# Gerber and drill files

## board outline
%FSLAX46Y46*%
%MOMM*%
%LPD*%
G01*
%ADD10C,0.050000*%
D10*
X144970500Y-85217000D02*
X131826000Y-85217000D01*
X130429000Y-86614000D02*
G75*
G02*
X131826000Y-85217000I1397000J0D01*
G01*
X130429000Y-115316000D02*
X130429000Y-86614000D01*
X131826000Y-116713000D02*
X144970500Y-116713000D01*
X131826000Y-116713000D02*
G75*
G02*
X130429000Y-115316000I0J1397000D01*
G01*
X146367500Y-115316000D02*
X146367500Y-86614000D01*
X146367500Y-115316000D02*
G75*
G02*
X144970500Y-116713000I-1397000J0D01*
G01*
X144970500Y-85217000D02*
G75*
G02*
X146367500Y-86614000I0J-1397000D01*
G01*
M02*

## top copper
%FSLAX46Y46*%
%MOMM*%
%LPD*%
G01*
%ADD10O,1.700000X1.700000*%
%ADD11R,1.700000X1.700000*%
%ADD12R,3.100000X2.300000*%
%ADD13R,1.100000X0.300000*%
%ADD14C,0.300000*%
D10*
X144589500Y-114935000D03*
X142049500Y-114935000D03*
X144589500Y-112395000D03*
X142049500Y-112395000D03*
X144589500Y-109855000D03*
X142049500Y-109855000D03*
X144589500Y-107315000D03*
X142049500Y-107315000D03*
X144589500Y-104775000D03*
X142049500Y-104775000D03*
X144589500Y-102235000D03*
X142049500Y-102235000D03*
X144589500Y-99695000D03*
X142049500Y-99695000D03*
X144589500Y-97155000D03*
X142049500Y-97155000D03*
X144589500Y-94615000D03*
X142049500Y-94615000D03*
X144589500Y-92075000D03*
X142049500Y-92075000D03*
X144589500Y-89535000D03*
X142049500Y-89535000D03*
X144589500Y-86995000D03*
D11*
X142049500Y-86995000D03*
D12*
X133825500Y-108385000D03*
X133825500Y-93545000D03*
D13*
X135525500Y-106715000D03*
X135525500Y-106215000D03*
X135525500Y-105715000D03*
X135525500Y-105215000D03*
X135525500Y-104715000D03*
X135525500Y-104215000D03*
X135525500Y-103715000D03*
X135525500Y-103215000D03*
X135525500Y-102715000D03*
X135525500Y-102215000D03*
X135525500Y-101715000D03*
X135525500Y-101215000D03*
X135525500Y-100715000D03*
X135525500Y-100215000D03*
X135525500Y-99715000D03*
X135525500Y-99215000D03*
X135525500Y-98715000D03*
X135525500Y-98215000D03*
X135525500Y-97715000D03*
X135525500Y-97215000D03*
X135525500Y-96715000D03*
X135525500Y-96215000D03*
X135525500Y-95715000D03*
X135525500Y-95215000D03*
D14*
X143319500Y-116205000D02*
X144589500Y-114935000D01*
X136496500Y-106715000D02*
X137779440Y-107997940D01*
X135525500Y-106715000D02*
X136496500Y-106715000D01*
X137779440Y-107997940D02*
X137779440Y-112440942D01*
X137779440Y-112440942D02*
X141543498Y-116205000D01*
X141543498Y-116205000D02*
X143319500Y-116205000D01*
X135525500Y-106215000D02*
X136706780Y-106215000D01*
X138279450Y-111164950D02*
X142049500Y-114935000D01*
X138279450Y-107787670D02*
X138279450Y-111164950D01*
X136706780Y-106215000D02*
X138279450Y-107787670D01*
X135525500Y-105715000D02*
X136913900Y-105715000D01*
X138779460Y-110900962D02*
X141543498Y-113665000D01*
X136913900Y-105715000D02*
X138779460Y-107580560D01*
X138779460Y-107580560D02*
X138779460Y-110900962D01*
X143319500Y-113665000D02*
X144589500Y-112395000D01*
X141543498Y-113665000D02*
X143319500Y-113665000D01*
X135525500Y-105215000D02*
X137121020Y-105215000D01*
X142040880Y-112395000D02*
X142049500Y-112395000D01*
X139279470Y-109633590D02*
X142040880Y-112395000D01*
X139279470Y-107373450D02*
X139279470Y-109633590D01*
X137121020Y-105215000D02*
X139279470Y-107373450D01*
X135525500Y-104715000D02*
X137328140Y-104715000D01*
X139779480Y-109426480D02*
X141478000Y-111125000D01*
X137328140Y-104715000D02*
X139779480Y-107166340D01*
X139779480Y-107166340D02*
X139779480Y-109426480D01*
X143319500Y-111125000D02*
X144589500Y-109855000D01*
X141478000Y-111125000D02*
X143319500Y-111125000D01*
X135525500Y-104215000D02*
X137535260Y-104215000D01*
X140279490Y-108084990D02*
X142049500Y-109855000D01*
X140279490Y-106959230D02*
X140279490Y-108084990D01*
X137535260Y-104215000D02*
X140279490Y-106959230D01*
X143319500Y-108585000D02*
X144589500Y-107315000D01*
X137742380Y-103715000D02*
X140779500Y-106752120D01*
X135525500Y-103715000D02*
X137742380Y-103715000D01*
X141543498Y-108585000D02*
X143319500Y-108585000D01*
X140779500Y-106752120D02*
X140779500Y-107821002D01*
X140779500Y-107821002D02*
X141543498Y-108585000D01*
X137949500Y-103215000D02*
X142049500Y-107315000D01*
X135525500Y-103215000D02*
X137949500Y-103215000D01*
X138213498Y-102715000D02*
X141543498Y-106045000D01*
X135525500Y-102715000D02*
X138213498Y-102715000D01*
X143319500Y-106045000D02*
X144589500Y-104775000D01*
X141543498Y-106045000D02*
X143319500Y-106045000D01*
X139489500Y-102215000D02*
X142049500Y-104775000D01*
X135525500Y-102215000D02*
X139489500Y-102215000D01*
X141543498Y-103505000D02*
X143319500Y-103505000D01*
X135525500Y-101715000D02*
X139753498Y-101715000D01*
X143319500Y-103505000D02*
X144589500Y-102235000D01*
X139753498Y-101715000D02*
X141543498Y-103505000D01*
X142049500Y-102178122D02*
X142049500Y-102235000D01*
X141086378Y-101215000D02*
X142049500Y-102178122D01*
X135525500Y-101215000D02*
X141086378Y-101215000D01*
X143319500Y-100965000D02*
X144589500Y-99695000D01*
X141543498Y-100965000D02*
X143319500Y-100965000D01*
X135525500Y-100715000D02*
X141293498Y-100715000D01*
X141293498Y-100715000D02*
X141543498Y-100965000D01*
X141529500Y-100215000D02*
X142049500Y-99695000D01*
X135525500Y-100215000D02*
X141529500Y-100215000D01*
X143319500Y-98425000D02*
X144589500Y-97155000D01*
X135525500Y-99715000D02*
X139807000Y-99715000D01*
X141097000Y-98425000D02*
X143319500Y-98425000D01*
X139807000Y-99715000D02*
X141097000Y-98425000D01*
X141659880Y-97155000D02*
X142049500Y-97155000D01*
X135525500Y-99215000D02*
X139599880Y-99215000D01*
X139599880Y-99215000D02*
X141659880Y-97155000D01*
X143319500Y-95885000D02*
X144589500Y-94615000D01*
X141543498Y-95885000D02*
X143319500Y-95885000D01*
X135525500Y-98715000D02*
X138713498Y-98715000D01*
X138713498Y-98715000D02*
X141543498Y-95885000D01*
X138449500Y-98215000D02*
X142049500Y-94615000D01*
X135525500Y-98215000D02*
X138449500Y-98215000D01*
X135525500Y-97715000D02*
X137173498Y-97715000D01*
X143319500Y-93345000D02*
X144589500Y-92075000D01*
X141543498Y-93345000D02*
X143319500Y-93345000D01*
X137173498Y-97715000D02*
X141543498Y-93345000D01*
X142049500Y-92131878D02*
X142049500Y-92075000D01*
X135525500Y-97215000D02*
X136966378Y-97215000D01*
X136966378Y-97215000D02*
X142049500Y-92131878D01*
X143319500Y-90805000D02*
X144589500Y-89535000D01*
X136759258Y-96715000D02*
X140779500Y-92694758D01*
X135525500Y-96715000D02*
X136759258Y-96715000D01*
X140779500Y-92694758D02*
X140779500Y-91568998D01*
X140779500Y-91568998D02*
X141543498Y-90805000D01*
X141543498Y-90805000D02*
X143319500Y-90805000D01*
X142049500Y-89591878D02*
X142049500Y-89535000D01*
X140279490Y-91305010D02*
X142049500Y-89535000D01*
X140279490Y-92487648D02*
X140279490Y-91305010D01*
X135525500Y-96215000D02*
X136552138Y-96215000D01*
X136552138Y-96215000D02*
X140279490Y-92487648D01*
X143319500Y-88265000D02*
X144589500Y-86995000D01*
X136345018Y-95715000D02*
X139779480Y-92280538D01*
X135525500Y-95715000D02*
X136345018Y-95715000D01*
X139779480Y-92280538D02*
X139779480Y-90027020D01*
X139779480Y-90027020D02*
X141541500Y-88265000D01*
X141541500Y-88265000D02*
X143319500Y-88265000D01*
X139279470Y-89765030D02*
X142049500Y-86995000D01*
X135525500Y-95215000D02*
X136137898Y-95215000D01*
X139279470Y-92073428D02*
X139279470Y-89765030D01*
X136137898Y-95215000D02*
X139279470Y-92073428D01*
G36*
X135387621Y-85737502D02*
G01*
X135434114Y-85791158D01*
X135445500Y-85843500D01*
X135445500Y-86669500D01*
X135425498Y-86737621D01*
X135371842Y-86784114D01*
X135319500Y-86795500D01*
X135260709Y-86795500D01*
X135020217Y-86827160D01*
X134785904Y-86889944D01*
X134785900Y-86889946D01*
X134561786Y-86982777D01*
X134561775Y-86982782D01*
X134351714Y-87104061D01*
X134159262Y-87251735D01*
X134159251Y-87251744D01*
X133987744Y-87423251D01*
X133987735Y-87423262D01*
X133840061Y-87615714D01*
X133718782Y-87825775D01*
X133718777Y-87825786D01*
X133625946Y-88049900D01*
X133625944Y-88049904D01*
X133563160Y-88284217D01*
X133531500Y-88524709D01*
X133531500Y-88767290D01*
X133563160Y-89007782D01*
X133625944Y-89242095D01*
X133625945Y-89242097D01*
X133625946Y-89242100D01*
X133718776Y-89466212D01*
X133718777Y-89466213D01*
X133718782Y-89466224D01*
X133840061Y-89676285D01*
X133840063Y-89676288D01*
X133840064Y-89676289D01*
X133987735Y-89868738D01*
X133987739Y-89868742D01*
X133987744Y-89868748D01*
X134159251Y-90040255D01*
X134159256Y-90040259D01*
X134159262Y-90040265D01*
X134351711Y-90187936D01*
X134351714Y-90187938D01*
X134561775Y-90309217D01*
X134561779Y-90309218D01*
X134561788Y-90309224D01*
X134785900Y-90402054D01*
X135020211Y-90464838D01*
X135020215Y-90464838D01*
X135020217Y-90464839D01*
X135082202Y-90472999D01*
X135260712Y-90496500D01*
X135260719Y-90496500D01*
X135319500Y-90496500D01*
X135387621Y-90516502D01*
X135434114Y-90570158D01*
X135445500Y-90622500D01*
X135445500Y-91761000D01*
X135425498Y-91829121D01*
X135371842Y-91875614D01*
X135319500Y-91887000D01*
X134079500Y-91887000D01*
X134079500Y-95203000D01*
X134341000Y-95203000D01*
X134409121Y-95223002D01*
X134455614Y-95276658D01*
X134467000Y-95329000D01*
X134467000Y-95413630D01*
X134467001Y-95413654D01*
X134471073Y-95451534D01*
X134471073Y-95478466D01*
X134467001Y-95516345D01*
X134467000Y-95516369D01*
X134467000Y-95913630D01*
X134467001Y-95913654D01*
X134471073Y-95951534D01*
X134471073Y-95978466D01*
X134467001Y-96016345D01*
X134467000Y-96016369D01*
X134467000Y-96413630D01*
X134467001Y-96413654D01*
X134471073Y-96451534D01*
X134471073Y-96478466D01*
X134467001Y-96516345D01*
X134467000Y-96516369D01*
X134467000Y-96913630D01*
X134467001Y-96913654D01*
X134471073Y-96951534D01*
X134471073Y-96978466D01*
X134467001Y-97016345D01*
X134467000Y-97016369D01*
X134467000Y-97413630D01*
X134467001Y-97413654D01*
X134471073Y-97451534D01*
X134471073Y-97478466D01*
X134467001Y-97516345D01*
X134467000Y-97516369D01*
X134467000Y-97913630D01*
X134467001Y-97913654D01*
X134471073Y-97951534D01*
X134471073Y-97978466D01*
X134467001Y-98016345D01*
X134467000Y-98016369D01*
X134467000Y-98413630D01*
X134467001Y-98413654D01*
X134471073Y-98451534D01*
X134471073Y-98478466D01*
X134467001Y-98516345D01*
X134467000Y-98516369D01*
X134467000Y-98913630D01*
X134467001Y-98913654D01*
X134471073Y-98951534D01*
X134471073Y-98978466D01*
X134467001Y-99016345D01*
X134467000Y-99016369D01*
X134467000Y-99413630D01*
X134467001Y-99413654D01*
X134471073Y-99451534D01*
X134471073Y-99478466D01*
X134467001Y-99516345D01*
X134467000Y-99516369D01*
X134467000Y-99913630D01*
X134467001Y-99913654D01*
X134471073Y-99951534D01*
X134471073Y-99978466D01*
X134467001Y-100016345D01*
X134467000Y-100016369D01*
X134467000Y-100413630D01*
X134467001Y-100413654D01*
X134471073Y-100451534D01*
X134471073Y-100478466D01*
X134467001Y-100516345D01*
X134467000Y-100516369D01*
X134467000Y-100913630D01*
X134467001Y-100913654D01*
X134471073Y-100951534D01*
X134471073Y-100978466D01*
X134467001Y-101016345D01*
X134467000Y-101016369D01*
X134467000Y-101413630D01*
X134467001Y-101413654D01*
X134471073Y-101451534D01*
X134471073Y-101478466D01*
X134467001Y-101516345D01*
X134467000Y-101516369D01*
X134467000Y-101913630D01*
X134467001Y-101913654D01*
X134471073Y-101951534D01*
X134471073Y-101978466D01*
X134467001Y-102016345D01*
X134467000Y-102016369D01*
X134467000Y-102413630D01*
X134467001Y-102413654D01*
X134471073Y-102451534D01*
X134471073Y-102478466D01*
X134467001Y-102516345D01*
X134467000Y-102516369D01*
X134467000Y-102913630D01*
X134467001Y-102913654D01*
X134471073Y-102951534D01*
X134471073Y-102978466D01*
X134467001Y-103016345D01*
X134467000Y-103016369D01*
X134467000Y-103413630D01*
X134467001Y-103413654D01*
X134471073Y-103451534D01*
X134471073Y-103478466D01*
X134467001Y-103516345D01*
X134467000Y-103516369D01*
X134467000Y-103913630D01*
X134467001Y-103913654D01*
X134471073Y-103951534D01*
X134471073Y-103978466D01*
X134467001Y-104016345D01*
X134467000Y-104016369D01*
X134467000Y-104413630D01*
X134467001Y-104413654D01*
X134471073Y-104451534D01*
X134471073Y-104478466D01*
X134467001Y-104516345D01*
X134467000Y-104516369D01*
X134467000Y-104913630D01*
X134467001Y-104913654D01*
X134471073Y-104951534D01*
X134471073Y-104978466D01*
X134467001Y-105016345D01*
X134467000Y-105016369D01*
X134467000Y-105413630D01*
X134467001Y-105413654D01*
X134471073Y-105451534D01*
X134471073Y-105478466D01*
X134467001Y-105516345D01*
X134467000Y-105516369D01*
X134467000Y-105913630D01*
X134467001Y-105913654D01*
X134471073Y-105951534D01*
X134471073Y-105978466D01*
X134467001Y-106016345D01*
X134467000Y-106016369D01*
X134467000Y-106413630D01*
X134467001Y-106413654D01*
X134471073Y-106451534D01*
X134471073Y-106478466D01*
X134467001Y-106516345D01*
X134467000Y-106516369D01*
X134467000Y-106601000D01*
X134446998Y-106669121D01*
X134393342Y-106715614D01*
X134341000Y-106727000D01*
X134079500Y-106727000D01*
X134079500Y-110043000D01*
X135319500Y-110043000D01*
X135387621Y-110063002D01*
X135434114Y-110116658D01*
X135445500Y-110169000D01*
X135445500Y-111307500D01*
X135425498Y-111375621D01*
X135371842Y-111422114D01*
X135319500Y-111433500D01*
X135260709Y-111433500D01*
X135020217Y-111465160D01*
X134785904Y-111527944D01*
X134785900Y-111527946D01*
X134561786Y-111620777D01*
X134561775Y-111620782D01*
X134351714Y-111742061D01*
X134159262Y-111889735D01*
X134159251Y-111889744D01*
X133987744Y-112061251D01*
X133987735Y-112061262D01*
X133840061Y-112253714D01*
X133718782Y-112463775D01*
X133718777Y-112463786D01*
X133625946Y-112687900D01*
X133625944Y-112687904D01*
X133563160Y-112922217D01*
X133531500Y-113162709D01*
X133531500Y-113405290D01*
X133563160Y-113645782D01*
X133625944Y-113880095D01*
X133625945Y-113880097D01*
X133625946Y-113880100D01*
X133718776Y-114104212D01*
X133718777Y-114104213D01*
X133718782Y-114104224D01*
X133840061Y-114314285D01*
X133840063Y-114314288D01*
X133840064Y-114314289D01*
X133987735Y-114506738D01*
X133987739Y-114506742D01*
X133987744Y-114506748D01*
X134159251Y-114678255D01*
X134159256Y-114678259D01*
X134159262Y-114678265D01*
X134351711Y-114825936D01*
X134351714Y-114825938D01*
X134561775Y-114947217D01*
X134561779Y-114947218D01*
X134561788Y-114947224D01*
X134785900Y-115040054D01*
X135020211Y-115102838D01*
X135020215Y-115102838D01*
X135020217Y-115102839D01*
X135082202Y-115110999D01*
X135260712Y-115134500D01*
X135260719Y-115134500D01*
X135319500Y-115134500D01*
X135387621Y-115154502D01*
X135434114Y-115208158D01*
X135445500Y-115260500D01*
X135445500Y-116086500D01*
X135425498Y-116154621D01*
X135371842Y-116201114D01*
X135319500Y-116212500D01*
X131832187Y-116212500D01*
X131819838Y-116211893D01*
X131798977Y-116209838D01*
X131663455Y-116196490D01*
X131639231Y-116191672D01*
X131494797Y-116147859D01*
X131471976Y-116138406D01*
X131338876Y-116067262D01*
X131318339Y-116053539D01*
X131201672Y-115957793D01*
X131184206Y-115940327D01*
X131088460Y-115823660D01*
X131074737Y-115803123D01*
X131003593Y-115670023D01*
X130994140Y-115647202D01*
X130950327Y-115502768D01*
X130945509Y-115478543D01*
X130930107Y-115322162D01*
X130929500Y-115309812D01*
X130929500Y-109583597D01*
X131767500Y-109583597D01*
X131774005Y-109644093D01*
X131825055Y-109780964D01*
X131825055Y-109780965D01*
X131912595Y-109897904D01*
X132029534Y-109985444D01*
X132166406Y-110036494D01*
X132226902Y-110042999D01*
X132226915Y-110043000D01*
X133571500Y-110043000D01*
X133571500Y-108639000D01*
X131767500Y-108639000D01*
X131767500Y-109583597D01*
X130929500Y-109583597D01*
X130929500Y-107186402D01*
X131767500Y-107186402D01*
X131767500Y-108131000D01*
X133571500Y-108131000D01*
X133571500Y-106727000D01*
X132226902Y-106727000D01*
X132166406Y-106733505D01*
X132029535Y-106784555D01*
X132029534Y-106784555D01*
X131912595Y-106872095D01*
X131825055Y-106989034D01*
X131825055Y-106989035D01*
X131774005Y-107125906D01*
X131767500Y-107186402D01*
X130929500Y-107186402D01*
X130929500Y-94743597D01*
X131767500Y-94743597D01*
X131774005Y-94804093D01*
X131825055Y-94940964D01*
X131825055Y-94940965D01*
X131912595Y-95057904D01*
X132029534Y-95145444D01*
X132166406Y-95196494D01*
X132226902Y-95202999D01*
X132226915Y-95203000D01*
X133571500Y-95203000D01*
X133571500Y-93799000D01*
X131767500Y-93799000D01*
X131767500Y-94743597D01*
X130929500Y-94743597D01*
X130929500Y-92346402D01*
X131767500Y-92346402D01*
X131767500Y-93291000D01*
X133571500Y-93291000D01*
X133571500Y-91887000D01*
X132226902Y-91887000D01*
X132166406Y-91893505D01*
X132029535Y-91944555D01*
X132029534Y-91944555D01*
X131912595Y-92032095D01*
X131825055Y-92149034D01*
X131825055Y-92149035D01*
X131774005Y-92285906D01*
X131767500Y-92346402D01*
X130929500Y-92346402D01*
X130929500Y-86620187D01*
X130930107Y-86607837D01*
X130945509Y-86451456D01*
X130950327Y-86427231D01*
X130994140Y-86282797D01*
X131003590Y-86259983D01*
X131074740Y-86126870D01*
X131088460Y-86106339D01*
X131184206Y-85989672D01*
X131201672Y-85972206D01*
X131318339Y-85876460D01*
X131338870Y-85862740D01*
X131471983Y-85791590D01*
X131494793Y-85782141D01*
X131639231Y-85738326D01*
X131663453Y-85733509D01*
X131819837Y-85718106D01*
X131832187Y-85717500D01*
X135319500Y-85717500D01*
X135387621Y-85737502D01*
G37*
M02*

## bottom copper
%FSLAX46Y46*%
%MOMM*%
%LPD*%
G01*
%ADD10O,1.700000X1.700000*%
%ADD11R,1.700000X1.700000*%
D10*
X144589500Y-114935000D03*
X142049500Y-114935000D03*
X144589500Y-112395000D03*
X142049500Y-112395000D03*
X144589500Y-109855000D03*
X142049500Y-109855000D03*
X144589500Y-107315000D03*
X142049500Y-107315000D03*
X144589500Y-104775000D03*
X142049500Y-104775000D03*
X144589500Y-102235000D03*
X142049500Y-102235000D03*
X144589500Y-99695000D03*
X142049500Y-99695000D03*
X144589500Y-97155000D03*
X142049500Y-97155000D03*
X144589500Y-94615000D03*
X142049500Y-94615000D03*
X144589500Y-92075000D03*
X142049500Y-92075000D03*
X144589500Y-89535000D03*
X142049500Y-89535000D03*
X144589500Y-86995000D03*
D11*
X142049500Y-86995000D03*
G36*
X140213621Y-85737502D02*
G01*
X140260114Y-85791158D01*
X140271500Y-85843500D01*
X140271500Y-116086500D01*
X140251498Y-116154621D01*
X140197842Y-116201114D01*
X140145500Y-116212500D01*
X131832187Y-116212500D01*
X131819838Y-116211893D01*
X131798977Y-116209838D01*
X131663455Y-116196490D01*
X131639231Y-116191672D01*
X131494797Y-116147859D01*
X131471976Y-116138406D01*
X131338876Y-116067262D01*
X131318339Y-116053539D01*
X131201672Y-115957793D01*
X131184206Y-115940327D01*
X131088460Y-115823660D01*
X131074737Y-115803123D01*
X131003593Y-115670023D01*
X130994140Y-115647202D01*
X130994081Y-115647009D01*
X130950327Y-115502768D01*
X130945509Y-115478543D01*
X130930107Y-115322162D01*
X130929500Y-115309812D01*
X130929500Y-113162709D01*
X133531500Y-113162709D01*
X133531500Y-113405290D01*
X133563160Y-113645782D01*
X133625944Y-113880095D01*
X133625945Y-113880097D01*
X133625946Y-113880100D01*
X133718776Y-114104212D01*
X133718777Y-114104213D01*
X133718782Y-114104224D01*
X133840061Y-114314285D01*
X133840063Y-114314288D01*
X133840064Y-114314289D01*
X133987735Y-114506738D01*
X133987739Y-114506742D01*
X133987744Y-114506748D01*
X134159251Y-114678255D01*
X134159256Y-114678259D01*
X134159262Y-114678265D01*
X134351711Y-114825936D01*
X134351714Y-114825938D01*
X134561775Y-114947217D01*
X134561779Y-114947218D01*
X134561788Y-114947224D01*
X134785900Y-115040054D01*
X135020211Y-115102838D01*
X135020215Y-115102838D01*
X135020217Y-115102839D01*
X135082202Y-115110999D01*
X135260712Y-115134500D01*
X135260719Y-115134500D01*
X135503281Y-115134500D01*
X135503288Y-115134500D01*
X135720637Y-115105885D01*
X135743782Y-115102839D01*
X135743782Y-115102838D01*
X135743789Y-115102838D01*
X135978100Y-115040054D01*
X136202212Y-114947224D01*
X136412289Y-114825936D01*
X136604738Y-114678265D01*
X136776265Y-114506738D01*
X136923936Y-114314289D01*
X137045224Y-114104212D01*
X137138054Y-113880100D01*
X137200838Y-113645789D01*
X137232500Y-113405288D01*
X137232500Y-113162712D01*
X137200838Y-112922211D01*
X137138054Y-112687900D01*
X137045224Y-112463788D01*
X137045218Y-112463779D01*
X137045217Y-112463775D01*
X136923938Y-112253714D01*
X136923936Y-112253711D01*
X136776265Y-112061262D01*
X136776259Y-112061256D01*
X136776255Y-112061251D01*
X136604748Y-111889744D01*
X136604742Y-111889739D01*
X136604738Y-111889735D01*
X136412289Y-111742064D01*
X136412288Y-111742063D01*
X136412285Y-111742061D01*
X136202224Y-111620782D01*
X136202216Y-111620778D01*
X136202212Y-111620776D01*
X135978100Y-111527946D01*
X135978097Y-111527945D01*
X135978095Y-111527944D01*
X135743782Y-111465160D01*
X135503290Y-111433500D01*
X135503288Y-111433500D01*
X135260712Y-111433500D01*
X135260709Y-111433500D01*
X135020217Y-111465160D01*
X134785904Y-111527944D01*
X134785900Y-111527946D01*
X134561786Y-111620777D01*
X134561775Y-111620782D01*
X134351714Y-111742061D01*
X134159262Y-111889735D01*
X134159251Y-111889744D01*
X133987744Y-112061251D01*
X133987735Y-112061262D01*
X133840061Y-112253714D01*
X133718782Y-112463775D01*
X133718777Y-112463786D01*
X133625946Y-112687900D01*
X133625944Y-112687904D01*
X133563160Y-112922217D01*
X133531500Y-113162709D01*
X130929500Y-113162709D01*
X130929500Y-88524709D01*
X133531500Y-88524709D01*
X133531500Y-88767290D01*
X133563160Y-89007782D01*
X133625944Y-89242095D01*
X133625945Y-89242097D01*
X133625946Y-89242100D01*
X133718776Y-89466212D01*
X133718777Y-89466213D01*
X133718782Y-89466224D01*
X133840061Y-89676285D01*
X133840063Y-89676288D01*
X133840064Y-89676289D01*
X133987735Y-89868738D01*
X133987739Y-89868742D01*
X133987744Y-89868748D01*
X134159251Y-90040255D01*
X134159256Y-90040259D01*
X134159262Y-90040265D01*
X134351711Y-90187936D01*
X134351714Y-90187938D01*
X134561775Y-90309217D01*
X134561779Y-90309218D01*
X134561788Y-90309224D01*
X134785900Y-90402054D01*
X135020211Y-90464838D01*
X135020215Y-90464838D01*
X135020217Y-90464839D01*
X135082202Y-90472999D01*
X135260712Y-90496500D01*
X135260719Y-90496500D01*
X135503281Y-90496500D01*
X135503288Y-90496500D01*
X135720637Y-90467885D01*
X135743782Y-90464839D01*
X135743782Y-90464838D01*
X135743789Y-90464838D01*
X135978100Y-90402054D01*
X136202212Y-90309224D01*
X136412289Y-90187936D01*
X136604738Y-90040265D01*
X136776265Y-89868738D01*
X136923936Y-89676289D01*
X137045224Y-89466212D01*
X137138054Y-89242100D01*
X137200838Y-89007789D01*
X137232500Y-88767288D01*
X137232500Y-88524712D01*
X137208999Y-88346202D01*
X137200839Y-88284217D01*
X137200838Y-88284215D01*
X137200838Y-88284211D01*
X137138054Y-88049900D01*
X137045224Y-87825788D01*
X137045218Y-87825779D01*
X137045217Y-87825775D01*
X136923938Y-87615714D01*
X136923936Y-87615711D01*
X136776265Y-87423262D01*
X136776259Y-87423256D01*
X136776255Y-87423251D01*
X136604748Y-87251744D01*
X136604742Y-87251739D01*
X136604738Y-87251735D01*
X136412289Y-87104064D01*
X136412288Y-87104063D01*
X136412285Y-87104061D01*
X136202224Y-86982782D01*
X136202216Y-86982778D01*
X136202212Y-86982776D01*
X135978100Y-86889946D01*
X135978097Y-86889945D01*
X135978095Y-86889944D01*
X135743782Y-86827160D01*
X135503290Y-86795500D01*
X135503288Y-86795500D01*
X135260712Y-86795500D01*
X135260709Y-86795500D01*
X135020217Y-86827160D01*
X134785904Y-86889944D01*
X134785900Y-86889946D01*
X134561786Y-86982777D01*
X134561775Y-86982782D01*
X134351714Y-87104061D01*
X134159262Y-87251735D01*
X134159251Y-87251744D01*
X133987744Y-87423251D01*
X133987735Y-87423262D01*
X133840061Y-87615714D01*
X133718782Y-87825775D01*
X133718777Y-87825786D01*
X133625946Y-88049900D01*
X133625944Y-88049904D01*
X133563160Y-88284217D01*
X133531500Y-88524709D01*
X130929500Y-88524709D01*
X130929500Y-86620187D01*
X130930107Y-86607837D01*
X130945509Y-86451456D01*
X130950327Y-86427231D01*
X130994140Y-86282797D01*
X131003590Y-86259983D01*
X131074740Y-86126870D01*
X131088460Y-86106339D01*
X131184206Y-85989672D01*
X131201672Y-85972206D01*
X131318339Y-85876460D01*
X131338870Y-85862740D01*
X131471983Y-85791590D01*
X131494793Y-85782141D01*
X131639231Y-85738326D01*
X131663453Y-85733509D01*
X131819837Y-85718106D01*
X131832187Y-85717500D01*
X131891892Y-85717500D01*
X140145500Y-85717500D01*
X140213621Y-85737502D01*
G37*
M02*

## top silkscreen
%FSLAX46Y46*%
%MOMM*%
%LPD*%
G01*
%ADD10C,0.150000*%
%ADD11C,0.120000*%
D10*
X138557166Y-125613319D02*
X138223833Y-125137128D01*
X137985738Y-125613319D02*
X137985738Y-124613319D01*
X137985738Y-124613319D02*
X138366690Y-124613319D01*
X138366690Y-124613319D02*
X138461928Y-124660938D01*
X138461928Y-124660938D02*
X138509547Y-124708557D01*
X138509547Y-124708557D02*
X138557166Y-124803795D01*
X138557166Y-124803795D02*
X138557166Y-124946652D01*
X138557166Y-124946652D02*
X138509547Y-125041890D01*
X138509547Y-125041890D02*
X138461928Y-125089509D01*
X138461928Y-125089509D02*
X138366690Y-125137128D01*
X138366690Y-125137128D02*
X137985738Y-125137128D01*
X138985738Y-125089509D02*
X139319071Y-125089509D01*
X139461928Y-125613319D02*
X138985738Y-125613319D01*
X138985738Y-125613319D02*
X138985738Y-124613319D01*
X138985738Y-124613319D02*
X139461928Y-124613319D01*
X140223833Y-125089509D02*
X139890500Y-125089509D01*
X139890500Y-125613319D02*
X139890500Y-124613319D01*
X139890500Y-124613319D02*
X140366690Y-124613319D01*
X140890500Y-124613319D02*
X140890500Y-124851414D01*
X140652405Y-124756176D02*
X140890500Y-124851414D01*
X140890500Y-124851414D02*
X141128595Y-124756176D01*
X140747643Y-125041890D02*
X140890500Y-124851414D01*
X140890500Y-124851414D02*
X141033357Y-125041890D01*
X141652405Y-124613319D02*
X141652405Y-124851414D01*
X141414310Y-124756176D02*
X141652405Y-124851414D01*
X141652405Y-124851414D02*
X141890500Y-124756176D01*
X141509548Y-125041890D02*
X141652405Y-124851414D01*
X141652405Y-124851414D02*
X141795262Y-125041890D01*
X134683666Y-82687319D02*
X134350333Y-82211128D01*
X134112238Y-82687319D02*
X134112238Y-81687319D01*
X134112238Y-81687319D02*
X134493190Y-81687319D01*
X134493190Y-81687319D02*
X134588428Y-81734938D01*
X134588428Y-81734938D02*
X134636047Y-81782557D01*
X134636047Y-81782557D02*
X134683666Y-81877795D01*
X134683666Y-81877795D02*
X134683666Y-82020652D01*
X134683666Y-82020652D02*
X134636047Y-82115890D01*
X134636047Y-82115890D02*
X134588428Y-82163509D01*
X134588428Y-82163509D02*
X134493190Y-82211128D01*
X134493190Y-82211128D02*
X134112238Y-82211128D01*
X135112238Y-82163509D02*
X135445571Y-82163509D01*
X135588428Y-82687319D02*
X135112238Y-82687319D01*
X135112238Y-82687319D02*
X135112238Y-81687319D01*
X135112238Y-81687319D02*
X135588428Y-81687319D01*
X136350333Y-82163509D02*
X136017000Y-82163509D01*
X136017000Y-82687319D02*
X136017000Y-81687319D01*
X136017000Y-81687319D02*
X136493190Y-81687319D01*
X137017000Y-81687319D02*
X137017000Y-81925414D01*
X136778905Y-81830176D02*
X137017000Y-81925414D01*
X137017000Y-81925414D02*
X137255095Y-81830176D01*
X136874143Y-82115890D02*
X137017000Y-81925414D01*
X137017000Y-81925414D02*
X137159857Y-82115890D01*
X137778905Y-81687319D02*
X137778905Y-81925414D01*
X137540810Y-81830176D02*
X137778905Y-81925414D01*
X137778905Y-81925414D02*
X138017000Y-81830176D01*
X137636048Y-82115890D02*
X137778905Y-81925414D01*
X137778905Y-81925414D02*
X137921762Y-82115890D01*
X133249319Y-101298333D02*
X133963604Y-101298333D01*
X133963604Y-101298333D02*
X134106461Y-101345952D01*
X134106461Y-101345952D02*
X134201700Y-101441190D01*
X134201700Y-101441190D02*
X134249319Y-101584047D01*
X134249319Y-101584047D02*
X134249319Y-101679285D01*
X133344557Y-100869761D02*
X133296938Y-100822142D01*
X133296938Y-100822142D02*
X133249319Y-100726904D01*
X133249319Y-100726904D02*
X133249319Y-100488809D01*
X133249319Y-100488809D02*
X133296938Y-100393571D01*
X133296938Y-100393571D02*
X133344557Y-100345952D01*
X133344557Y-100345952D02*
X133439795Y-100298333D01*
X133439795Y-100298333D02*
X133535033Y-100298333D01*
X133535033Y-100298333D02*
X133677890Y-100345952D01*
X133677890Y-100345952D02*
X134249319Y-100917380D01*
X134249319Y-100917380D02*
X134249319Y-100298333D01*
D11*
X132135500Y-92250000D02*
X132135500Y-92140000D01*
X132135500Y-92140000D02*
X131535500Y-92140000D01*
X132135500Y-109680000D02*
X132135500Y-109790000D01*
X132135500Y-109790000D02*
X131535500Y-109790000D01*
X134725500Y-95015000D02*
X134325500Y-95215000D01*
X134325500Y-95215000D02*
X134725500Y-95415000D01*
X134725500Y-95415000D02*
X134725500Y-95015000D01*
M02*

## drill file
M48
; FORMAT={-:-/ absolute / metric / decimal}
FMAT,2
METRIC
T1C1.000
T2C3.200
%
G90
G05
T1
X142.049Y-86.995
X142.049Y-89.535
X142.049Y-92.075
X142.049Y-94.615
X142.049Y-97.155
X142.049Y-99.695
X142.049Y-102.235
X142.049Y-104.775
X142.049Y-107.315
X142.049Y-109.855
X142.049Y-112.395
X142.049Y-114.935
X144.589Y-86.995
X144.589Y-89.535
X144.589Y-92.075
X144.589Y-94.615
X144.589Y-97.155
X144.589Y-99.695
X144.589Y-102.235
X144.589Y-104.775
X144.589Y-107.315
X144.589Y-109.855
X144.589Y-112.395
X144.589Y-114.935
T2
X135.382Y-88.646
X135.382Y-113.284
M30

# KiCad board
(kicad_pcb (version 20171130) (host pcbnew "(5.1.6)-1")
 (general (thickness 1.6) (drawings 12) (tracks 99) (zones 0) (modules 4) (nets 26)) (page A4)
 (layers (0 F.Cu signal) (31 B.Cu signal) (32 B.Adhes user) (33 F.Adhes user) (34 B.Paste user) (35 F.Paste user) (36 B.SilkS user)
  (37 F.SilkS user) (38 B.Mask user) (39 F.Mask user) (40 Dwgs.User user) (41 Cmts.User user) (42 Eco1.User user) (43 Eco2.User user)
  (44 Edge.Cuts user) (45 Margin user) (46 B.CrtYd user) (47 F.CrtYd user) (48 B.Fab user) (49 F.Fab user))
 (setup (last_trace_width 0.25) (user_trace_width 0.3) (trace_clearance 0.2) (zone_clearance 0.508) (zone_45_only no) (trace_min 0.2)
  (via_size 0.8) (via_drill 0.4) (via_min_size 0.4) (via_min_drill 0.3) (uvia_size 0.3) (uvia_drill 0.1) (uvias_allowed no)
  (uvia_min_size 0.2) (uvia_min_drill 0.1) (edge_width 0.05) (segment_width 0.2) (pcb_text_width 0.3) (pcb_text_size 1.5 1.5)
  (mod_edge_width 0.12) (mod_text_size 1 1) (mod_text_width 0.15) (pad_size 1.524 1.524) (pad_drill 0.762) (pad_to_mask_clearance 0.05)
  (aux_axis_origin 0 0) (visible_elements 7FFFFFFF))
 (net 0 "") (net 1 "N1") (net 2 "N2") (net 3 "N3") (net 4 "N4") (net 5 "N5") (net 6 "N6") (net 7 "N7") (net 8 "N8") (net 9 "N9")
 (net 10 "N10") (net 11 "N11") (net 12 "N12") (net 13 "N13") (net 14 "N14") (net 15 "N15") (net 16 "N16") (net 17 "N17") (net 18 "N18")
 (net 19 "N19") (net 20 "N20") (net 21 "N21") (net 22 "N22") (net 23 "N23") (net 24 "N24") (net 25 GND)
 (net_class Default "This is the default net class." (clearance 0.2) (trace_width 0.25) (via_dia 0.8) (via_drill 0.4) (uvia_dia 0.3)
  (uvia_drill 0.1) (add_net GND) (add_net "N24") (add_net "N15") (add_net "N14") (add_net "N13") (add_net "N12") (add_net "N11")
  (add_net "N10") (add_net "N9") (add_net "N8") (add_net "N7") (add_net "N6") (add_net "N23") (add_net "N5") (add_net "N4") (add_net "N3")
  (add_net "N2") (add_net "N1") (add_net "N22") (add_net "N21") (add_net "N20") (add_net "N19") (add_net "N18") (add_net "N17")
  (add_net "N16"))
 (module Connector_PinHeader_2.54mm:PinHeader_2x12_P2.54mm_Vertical (layer F.Cu) (at 142.0495 86.995)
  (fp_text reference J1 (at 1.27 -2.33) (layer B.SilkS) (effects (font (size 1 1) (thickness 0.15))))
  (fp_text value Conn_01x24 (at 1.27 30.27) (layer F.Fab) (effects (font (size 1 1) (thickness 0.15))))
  (pad 24 thru_hole oval (at 2.54 27.94) (size 1.7 1.7) (drill 1) (layers *.Cu *.Mask) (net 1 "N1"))
  (pad 23 thru_hole oval (at 0 27.94) (size 1.7 1.7) (drill 1) (layers *.Cu *.Mask) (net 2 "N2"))
  (pad 22 thru_hole oval (at 2.54 25.4) (size 1.7 1.7) (drill 1) (layers *.Cu *.Mask) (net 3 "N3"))
  (pad 21 thru_hole oval (at 0 25.4) (size 1.7 1.7) (drill 1) (layers *.Cu *.Mask) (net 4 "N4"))
  (pad 20 thru_hole oval (at 2.54 22.86) (size 1.7 1.7) (drill 1) (layers *.Cu *.Mask) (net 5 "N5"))
  (pad 19 thru_hole oval (at 0 22.86) (size 1.7 1.7) (drill 1) (layers *.Cu *.Mask) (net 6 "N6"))
  (pad 18 thru_hole oval (at 2.54 20.32) (size 1.7 1.7) (drill 1) (layers *.Cu *.Mask) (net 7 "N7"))
  (pad 17 thru_hole oval (at 0 20.32) (size 1.7 1.7) (drill 1) (layers *.Cu *.Mask) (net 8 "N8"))
  (pad 16 thru_hole oval (at 2.54 17.78) (size 1.7 1.7) (drill 1) (layers *.Cu *.Mask) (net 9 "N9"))
  (pad 15 thru_hole oval (at 0 17.78) (size 1.7 1.7) (drill 1) (layers *.Cu *.Mask) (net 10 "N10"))
  (pad 14 thru_hole oval (at 2.54 15.24) (size 1.7 1.7) (drill 1) (layers *.Cu *.Mask) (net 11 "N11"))
  (pad 13 thru_hole oval (at 0 15.24) (size 1.7 1.7) (drill 1) (layers *.Cu *.Mask) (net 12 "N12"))
  (pad 12 thru_hole oval (at 2.54 12.7) (size 1.7 1.7) (drill 1) (layers *.Cu *.Mask) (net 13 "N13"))
  (pad 11 thru_hole oval (at 0 12.7) (size 1.7 1.7) (drill 1) (layers *.Cu *.Mask) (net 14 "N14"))
  (pad 10 thru_hole oval (at 2.54 10.16) (size 1.7 1.7) (drill 1) (layers *.Cu *.Mask) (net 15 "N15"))
  (pad 9 thru_hole oval (at 0 10.16) (size 1.7 1.7) (drill 1) (layers *.Cu *.Mask) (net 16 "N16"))
  (pad 8 thru_hole oval (at 2.54 7.62) (size 1.7 1.7) (drill 1) (layers *.Cu *.Mask) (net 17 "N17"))
  (pad 7 thru_hole oval (at 0 7.62) (size 1.7 1.7) (drill 1) (layers *.Cu *.Mask) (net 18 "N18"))
  (pad 6 thru_hole oval (at 2.54 5.08) (size 1.7 1.7) (drill 1) (layers *.Cu *.Mask) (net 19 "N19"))
  (pad 5 thru_hole oval (at 0 5.08) (size 1.7 1.7) (drill 1) (layers *.Cu *.Mask) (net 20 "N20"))
  (pad 4 thru_hole oval (at 2.54 2.54) (size 1.7 1.7) (drill 1) (layers *.Cu *.Mask) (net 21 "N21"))
  (pad 3 thru_hole oval (at 0 2.54) (size 1.7 1.7) (drill 1) (layers *.Cu *.Mask) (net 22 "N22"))
  (pad 2 thru_hole oval (at 2.54 0) (size 1.7 1.7) (drill 1) (layers *.Cu *.Mask) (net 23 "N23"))
  (pad 1 thru_hole rect (at 0 0) (size 1.7 1.7) (drill 1) (layers *.Cu *.Mask) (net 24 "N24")))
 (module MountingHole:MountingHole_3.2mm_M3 (layer F.Cu) (at 135.382 113.284)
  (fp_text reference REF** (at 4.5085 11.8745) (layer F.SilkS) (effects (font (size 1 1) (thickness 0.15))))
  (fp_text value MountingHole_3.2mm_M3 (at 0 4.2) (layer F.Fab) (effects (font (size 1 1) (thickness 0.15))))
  (pad 1 np_thru_hole circle (at 0 0) (size 3.2 3.2) (drill 3.2) (layers *.Cu *.Mask)))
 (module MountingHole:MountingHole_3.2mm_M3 (layer F.Cu) (at 135.382 88.646)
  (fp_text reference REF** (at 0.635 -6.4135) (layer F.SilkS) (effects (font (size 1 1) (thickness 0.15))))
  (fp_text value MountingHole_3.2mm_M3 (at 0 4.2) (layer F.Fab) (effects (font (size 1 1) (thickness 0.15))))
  (pad 1 np_thru_hole circle (at 0 0) (size 3.2 3.2) (drill 3.2) (layers *.Cu *.Mask)))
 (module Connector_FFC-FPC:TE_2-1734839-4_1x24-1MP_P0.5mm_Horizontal (layer F.Cu) (at 134.1755 100.965 270)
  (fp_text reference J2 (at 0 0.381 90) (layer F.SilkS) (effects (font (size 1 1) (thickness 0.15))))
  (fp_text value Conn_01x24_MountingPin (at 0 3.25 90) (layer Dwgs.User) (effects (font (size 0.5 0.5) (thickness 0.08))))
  (fp_line (start -8.715 2.04) (end -8.825 2.04) (layer F.SilkS) (width 0.12))
  (fp_line (start -8.825 2.04) (end -8.825 2.64) (layer F.SilkS) (width 0.12))
  (fp_line (start 8.715 2.04) (end 8.825 2.04) (layer F.SilkS) (width 0.12))
  (fp_line (start 8.825 2.04) (end 8.825 2.64) (layer F.SilkS) (width 0.12))
  (fp_line (start -5.95 -0.55) (end -5.75 -0.15) (layer F.SilkS) (width 0.12))
  (fp_line (start -5.75 -0.15) (end -5.55 -0.55) (layer F.SilkS) (width 0.12))
  (fp_line (start -5.55 -0.55) (end -5.95 -0.55) (layer F.SilkS) (width 0.12))
  (pad MP smd rect (at 7.42 0.35 270) (size 2.3 3.1) (layers F.Cu F.Paste F.Mask) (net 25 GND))
  (pad MP smd rect (at -7.42 0.35 270) (size 2.3 3.1) (layers F.Cu F.Paste F.Mask) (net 25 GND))
  (pad 24 smd rect (at 5.75 -1.35 270) (size 0.3 1.1) (layers F.Cu F.Paste F.Mask) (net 1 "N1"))
  (pad 23 smd rect (at 5.25 -1.35 270) (size 0.3 1.1) (layers F.Cu F.Paste F.Mask) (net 2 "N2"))
  (pad 22 smd rect (at 4.75 -1.35 270) (size 0.3 1.1) (layers F.Cu F.Paste F.Mask) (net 3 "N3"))
  (pad 21 smd rect (at 4.25 -1.35 270) (size 0.3 1.1) (layers F.Cu F.Paste F.Mask) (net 4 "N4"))
  (pad 20 smd rect (at 3.75 -1.35 270) (size 0.3 1.1) (layers F.Cu F.Paste F.Mask) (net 5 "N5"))
  (pad 19 smd rect (at 3.25 -1.35 270) (size 0.3 1.1) (layers F.Cu F.Paste F.Mask) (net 6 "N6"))
  (pad 18 smd rect (at 2.75 -1.35 270) (size 0.3 1.1) (layers F.Cu F.Paste F.Mask) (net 7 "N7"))
  (pad 17 smd rect (at 2.25 -1.35 270) (size 0.3 1.1) (layers F.Cu F.Paste F.Mask) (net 8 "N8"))
  (pad 16 smd rect (at 1.75 -1.35 270) (size 0.3 1.1) (layers F.Cu F.Paste F.Mask) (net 9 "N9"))
  (pad 15 smd rect (at 1.25 -1.35 270) (size 0.3 1.1) (layers F.Cu F.Paste F.Mask) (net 10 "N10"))
  (pad 14 smd rect (at 0.75 -1.35 270) (size 0.3 1.1) (layers F.Cu F.Paste F.Mask) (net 11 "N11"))
  (pad 13 smd rect (at 0.25 -1.35 270) (size 0.3 1.1) (layers F.Cu F.Paste F.Mask) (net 12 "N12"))
  (pad 12 smd rect (at -0.25 -1.35 270) (size 0.3 1.1) (layers F.Cu F.Paste F.Mask) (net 13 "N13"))
  (pad 11 smd rect (at -0.75 -1.35 270) (size 0.3 1.1) (layers F.Cu F.Paste F.Mask) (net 14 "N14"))
  (pad 10 smd rect (at -1.25 -1.35 270) (size 0.3 1.1) (layers F.Cu F.Paste F.Mask) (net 15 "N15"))
  (pad 9 smd rect (at -1.75 -1.35 270) (size 0.3 1.1) (layers F.Cu F.Paste F.Mask) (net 16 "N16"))
  (pad 8 smd rect (at -2.25 -1.35 270) (size 0.3 1.1) (layers F.Cu F.Paste F.Mask) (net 17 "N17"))
  (pad 7 smd rect (at -2.75 -1.35 270) (size 0.3 1.1) (layers F.Cu F.Paste F.Mask) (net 18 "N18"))
  (pad 6 smd rect (at -3.25 -1.35 270) (size 0.3 1.1) (layers F.Cu F.Paste F.Mask) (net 19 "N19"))
  (pad 5 smd rect (at -3.75 -1.35 270) (size 0.3 1.1) (layers F.Cu F.Paste F.Mask) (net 20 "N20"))
  (pad 4 smd rect (at -4.25 -1.35 270) (size 0.3 1.1) (layers F.Cu F.Paste F.Mask) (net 21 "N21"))
  (pad 3 smd rect (at -4.75 -1.35 270) (size 0.3 1.1) (layers F.Cu F.Paste F.Mask) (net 22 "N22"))
  (pad 2 smd rect (at -5.25 -1.35 270) (size 0.3 1.1) (layers F.Cu F.Paste F.Mask) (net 23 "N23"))
  (pad 1 smd rect (at -5.75 -1.35 270) (size 0.3 1.1) (layers F.Cu F.Paste F.Mask) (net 24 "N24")))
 (gr_line (start 144.9705 85.217) (end 131.826 85.217) (layer Edge.Cuts) (width 0.05))
 (gr_arc (start 131.826 86.614) (end 131.826 85.217) (angle -90) (layer Edge.Cuts) (width 0.05))
 (gr_line (start 130.429 115.316) (end 130.429 86.614) (layer Edge.Cuts) (width 0.05))
 (gr_line (start 131.826 116.713) (end 144.9705 116.713) (layer Edge.Cuts) (width 0.05))
 (gr_arc (start 131.826 115.316) (end 130.429 115.316) (angle -90) (layer Edge.Cuts) (width 0.05))
 (gr_line (start 146.3675 115.316) (end 146.3675 86.614) (layer Edge.Cuts) (width 0.05))
 (gr_arc (start 144.9705 115.316) (end 144.9705 116.713) (angle -90) (layer Edge.Cuts) (width 0.05))
 (gr_arc (start 144.9705 86.614) (end 146.3675 86.614) (angle -90) (layer Edge.Cuts) (width 0.05))
 (segment (start 143.3195 116.205) (end 144.5895 114.935) (width 0.3) (layer F.Cu) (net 1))
 (segment (start 136.4965 106.715) (end 137.77944 107.99794) (width 0.3) (layer F.Cu) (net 1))
 (segment (start 135.5255 106.715) (end 136.4965 106.715) (width 0.3) (layer F.Cu) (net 1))
 (segment (start 137.77944 107.99794) (end 137.77944 112.440942) (width 0.3) (layer F.Cu) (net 1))
 (segment (start 137.77944 112.440942) (end 141.543498 116.205) (width 0.3) (layer F.Cu) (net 1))
 (segment (start 141.543498 116.205) (end 143.3195 116.205) (width 0.3) (layer F.Cu) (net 1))
 (segment (start 135.5255 106.215) (end 136.70678 106.215) (width 0.3) (layer F.Cu) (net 2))
 (segment (start 138.27945 111.16495) (end 142.0495 114.935) (width 0.3) (layer F.Cu) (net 2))
 (segment (start 138.27945 107.78767) (end 138.27945 111.16495) (width 0.3) (layer F.Cu) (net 2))
 (segment (start 136.70678 106.215) (end 138.27945 107.78767) (width 0.3) (layer F.Cu) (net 2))
 (segment (start 135.5255 105.715) (end 136.9139 105.715) (width 0.3) (layer F.Cu) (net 3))
 (segment (start 138.77946 110.900962) (end 141.543498 113.665) (width 0.3) (layer F.Cu) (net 3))
 (segment (start 136.9139 105.715) (end 138.77946 107.58056) (width 0.3) (layer F.Cu) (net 3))
 (segment (start 138.77946 107.58056) (end 138.77946 110.900962) (width 0.3) (layer F.Cu) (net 3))
 (segment (start 143.3195 113.665) (end 144.5895 112.395) (width 0.3) (layer F.Cu) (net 3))
 (segment (start 141.543498 113.665) (end 143.3195 113.665) (width 0.3) (layer F.Cu) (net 3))
 (segment (start 135.5255 105.215) (end 137.12102 105.215) (width 0.3) (layer F.Cu) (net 4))
 (segment (start 142.04088 112.395) (end 142.0495 112.395) (width 0.3) (layer F.Cu) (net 4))
 (segment (start 139.27947 109.63359) (end 142.04088 112.395) (width 0.3) (layer F.Cu) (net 4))
 (segment (start 139.27947 107.37345) (end 139.27947 109.63359) (width 0.3) (layer F.Cu) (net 4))
 (segment (start 137.12102 105.215) (end 139.27947 107.37345) (width 0.3) (layer F.Cu) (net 4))
 (segment (start 135.5255 104.715) (end 137.32814 104.715) (width 0.3) (layer F.Cu) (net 5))
 (segment (start 139.77948 109.42648) (end 141.478 111.125) (width 0.3) (layer F.Cu) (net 5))
 (segment (start 137.32814 104.715) (end 139.77948 107.16634) (width 0.3) (layer F.Cu) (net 5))
 (segment (start 139.77948 107.16634) (end 139.77948 109.42648) (width 0.3) (layer F.Cu) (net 5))
 (segment (start 143.3195 111.125) (end 144.5895 109.855) (width 0.3) (layer F.Cu) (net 5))
 (segment (start 141.478 111.125) (end 143.3195 111.125) (width 0.3) (layer F.Cu) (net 5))
 (segment (start 135.5255 104.215) (end 137.53526 104.215) (width 0.3) (layer F.Cu) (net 6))
 (segment (start 140.27949 108.08499) (end 142.0495 109.855) (width 0.3) (layer F.Cu) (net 6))
 (segment (start 140.27949 106.95923) (end 140.27949 108.08499) (width 0.3) (layer F.Cu) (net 6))
 (segment (start 137.53526 104.215) (end 140.27949 106.95923) (width 0.3) (layer F.Cu) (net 6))
 (segment (start 143.3195 108.585) (end 144.5895 107.315) (width 0.3) (layer F.Cu) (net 7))
 (segment (start 137.74238 103.715) (end 140.7795 106.75212) (width 0.3) (layer F.Cu) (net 7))
 (segment (start 135.5255 103.715) (end 137.74238 103.715) (width 0.3) (layer F.Cu) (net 7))
 (segment (start 141.543498 108.585) (end 143.3195 108.585) (width 0.3) (layer F.Cu) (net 7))
 (segment (start 140.7795 106.75212) (end 140.7795 107.821002) (width 0.3) (layer F.Cu) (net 7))
 (segment (start 140.7795 107.821002) (end 141.543498 108.585) (width 0.3) (layer F.Cu) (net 7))
 (segment (start 137.9495 103.215) (end 142.0495 107.315) (width 0.3) (layer F.Cu) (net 8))
 (segment (start 135.5255 103.215) (end 137.9495 103.215) (width 0.3) (layer F.Cu) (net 8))
 (segment (start 138.213498 102.715) (end 141.543498 106.045) (width 0.3) (layer F.Cu) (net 9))
 (segment (start 135.5255 102.715) (end 138.213498 102.715) (width 0.3) (layer F.Cu) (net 9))
 (segment (start 143.3195 106.045) (end 144.5895 104.775) (width 0.3) (layer F.Cu) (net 9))
 (segment (start 141.543498 106.045) (end 143.3195 106.045) (width 0.3) (layer F.Cu) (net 9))
 (segment (start 139.4895 102.215) (end 142.0495 104.775) (width 0.3) (layer F.Cu) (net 10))
 (segment (start 135.5255 102.215) (end 139.4895 102.215) (width 0.3) (layer F.Cu) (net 10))
 (segment (start 141.543498 103.505) (end 143.3195 103.505) (width 0.3) (layer F.Cu) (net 11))
 (segment (start 135.5255 101.715) (end 139.753498 101.715) (width 0.3) (layer F.Cu) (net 11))
 (segment (start 143.3195 103.505) (end 144.5895 102.235) (width 0.3) (layer F.Cu) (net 11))
 (segment (start 139.753498 101.715) (end 141.543498 103.505) (width 0.3) (layer F.Cu) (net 11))
 (segment (start 142.0495 102.178122) (end 142.0495 102.235) (width 0.3) (layer F.Cu) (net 12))
 (segment (start 141.086378 101.215) (end 142.0495 102.178122) (width 0.3) (layer F.Cu) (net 12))
 (segment (start 135.5255 101.215) (end 141.086378 101.215) (width 0.3) (layer F.Cu) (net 12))
 (segment (start 143.3195 100.965) (end 144.5895 99.695) (width 0.3) (layer F.Cu) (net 13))
 (segment (start 141.543498 100.965) (end 143.3195 100.965) (width 0.3) (layer F.Cu) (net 13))
 (segment (start 135.5255 100.715) (end 141.293498 100.715) (width 0.3) (layer F.Cu) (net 13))
 (segment (start 141.293498 100.715) (end 141.543498 100.965) (width 0.3) (layer F.Cu) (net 13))
 (segment (start 141.5295 100.215) (end 142.0495 99.695) (width 0.3) (layer F.Cu) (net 14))
 (segment (start 135.5255 100.215) (end 141.5295 100.215) (width 0.3) (layer F.Cu) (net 14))
 (segment (start 143.3195 98.425) (end 144.5895 97.155) (width 0.3) (layer F.Cu) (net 15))
 (segment (start 135.5255 99.715) (end 139.807 99.715) (width 0.3) (layer F.Cu) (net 15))
 (segment (start 141.097 98.425) (end 143.3195 98.425) (width 0.3) (layer F.Cu) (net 15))
 (segment (start 139.807 99.715) (end 141.097 98.425) (width 0.3) (layer F.Cu) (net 15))
 (segment (start 141.65988 97.155) (end 142.0495 97.155) (width 0.3) (layer F.Cu) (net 16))
 (segment (start 135.5255 99.215) (end 139.59988 99.215) (width 0.3) (layer F.Cu) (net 16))
 (segment (start 139.59988 99.215) (end 141.65988 97.155) (width 0.3) (layer F.Cu) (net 16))
 (segment (start 143.3195 95.885) (end 144.5895 94.615) (width 0.3) (layer F.Cu) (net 17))
 (segment (start 141.543498 95.885) (end 143.3195 95.885) (width 0.3) (layer F.Cu) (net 17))
 (segment (start 135.5255 98.715) (end 138.713498 98.715) (width 0.3) (layer F.Cu) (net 17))
 (segment (start 138.713498 98.715) (end 141.543498 95.885) (width 0.3) (layer F.Cu) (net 17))
 (segment (start 138.4495 98.215) (end 142.0495 94.615) (width 0.3) (layer F.Cu) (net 18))
 (segment (start 135.5255 98.215) (end 138.4495 98.215) (width 0.3) (layer F.Cu) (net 18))
 (segment (start 135.5255 97.715) (end 137.173498 97.715) (width 0.3) (layer F.Cu) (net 19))
 (segment (start 143.3195 93.345) (end 144.5895 92.075) (width 0.3) (layer F.Cu) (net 19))
 (segment (start 141.543498 93.345) (end 143.3195 93.345) (width 0.3) (layer F.Cu) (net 19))
 (segment (start 137.173498 97.715) (end 141.543498 93.345) (width 0.3) (layer F.Cu) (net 19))
 (segment (start 142.0495 92.131878) (end 142.0495 92.075) (width 0.3) (layer F.Cu) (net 20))
 (segment (start 135.5255 97.215) (end 136.966378 97.215) (width 0.3) (layer F.Cu) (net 20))
 (segment (start 136.966378 97.215) (end 142.0495 92.131878) (width 0.3) (layer F.Cu) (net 20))
 (segment (start 143.3195 90.805) (end 144.5895 89.535) (width 0.3) (layer F.Cu) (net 21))
 (segment (start 136.759258 96.715) (end 140.7795 92.694758) (width 0.3) (layer F.Cu) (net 21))
 (segment (start 135.5255 96.715) (end 136.759258 96.715) (width 0.3) (layer F.Cu) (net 21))
 (segment (start 140.7795 92.694758) (end 140.7795 91.568998) (width 0.3) (layer F.Cu) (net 21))
 (segment (start 140.7795 91.568998) (end 141.543498 90.805) (width 0.3) (layer F.Cu) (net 21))
 (segment (start 141.543498 90.805) (end 143.3195 90.805) (width 0.3) (layer F.Cu) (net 21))
 (segment (start 142.0495 89.591878) (end 142.0495 89.535) (width 0.3) (layer F.Cu) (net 22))
 (segment (start 140.27949 91.30501) (end 142.0495 89.535) (width 0.3) (layer F.Cu) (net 22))
 (segment (start 140.27949 92.487648) (end 140.27949 91.30501) (width 0.3) (layer F.Cu) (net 22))
 (segment (start 135.5255 96.215) (end 136.552138 96.215) (width 0.3) (layer F.Cu) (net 22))
 (segment (start 136.552138 96.215) (end 140.27949 92.487648) (width 0.3) (layer F.Cu) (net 22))
 (segment (start 143.3195 88.265) (end 144.5895 86.995) (width 0.3) (layer F.Cu) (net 23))
 (segment (start 136.345018 95.715) (end 139.77948 92.280538) (width 0.3) (layer F.Cu) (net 23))
 (segment (start 135.5255 95.715) (end 136.345018 95.715) (width 0.3) (layer F.Cu) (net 23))
 (segment (start 139.77948 92.280538) (end 139.77948 90.02702) (width 0.3) (layer F.Cu) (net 23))
 (segment (start 139.77948 90.02702) (end 141.5415 88.265) (width 0.3) (layer F.Cu) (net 23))
 (segment (start 141.5415 88.265) (end 143.3195 88.265) (width 0.3) (layer F.Cu) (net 23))
 (segment (start 139.27947 89.76503) (end 142.0495 86.995) (width 0.3) (layer F.Cu) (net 24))
 (segment (start 135.5255 95.215) (end 136.137898 95.215) (width 0.3) (layer F.Cu) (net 24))
 (segment (start 139.27947 92.073428) (end 139.27947 89.76503) (width 0.3) (layer F.Cu) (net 24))
 (segment (start 136.137898 95.215) (end 139.27947 92.073428) (width 0.3) (layer F.Cu) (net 24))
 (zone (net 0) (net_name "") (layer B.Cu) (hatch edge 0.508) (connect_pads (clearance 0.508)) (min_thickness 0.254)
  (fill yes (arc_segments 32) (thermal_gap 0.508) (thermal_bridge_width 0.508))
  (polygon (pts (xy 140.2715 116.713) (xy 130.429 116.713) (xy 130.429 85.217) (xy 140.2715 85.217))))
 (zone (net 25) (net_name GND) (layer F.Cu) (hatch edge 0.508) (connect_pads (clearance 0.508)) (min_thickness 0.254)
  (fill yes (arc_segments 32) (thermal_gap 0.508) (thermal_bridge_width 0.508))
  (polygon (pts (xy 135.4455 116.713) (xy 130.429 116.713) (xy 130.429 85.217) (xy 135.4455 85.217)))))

